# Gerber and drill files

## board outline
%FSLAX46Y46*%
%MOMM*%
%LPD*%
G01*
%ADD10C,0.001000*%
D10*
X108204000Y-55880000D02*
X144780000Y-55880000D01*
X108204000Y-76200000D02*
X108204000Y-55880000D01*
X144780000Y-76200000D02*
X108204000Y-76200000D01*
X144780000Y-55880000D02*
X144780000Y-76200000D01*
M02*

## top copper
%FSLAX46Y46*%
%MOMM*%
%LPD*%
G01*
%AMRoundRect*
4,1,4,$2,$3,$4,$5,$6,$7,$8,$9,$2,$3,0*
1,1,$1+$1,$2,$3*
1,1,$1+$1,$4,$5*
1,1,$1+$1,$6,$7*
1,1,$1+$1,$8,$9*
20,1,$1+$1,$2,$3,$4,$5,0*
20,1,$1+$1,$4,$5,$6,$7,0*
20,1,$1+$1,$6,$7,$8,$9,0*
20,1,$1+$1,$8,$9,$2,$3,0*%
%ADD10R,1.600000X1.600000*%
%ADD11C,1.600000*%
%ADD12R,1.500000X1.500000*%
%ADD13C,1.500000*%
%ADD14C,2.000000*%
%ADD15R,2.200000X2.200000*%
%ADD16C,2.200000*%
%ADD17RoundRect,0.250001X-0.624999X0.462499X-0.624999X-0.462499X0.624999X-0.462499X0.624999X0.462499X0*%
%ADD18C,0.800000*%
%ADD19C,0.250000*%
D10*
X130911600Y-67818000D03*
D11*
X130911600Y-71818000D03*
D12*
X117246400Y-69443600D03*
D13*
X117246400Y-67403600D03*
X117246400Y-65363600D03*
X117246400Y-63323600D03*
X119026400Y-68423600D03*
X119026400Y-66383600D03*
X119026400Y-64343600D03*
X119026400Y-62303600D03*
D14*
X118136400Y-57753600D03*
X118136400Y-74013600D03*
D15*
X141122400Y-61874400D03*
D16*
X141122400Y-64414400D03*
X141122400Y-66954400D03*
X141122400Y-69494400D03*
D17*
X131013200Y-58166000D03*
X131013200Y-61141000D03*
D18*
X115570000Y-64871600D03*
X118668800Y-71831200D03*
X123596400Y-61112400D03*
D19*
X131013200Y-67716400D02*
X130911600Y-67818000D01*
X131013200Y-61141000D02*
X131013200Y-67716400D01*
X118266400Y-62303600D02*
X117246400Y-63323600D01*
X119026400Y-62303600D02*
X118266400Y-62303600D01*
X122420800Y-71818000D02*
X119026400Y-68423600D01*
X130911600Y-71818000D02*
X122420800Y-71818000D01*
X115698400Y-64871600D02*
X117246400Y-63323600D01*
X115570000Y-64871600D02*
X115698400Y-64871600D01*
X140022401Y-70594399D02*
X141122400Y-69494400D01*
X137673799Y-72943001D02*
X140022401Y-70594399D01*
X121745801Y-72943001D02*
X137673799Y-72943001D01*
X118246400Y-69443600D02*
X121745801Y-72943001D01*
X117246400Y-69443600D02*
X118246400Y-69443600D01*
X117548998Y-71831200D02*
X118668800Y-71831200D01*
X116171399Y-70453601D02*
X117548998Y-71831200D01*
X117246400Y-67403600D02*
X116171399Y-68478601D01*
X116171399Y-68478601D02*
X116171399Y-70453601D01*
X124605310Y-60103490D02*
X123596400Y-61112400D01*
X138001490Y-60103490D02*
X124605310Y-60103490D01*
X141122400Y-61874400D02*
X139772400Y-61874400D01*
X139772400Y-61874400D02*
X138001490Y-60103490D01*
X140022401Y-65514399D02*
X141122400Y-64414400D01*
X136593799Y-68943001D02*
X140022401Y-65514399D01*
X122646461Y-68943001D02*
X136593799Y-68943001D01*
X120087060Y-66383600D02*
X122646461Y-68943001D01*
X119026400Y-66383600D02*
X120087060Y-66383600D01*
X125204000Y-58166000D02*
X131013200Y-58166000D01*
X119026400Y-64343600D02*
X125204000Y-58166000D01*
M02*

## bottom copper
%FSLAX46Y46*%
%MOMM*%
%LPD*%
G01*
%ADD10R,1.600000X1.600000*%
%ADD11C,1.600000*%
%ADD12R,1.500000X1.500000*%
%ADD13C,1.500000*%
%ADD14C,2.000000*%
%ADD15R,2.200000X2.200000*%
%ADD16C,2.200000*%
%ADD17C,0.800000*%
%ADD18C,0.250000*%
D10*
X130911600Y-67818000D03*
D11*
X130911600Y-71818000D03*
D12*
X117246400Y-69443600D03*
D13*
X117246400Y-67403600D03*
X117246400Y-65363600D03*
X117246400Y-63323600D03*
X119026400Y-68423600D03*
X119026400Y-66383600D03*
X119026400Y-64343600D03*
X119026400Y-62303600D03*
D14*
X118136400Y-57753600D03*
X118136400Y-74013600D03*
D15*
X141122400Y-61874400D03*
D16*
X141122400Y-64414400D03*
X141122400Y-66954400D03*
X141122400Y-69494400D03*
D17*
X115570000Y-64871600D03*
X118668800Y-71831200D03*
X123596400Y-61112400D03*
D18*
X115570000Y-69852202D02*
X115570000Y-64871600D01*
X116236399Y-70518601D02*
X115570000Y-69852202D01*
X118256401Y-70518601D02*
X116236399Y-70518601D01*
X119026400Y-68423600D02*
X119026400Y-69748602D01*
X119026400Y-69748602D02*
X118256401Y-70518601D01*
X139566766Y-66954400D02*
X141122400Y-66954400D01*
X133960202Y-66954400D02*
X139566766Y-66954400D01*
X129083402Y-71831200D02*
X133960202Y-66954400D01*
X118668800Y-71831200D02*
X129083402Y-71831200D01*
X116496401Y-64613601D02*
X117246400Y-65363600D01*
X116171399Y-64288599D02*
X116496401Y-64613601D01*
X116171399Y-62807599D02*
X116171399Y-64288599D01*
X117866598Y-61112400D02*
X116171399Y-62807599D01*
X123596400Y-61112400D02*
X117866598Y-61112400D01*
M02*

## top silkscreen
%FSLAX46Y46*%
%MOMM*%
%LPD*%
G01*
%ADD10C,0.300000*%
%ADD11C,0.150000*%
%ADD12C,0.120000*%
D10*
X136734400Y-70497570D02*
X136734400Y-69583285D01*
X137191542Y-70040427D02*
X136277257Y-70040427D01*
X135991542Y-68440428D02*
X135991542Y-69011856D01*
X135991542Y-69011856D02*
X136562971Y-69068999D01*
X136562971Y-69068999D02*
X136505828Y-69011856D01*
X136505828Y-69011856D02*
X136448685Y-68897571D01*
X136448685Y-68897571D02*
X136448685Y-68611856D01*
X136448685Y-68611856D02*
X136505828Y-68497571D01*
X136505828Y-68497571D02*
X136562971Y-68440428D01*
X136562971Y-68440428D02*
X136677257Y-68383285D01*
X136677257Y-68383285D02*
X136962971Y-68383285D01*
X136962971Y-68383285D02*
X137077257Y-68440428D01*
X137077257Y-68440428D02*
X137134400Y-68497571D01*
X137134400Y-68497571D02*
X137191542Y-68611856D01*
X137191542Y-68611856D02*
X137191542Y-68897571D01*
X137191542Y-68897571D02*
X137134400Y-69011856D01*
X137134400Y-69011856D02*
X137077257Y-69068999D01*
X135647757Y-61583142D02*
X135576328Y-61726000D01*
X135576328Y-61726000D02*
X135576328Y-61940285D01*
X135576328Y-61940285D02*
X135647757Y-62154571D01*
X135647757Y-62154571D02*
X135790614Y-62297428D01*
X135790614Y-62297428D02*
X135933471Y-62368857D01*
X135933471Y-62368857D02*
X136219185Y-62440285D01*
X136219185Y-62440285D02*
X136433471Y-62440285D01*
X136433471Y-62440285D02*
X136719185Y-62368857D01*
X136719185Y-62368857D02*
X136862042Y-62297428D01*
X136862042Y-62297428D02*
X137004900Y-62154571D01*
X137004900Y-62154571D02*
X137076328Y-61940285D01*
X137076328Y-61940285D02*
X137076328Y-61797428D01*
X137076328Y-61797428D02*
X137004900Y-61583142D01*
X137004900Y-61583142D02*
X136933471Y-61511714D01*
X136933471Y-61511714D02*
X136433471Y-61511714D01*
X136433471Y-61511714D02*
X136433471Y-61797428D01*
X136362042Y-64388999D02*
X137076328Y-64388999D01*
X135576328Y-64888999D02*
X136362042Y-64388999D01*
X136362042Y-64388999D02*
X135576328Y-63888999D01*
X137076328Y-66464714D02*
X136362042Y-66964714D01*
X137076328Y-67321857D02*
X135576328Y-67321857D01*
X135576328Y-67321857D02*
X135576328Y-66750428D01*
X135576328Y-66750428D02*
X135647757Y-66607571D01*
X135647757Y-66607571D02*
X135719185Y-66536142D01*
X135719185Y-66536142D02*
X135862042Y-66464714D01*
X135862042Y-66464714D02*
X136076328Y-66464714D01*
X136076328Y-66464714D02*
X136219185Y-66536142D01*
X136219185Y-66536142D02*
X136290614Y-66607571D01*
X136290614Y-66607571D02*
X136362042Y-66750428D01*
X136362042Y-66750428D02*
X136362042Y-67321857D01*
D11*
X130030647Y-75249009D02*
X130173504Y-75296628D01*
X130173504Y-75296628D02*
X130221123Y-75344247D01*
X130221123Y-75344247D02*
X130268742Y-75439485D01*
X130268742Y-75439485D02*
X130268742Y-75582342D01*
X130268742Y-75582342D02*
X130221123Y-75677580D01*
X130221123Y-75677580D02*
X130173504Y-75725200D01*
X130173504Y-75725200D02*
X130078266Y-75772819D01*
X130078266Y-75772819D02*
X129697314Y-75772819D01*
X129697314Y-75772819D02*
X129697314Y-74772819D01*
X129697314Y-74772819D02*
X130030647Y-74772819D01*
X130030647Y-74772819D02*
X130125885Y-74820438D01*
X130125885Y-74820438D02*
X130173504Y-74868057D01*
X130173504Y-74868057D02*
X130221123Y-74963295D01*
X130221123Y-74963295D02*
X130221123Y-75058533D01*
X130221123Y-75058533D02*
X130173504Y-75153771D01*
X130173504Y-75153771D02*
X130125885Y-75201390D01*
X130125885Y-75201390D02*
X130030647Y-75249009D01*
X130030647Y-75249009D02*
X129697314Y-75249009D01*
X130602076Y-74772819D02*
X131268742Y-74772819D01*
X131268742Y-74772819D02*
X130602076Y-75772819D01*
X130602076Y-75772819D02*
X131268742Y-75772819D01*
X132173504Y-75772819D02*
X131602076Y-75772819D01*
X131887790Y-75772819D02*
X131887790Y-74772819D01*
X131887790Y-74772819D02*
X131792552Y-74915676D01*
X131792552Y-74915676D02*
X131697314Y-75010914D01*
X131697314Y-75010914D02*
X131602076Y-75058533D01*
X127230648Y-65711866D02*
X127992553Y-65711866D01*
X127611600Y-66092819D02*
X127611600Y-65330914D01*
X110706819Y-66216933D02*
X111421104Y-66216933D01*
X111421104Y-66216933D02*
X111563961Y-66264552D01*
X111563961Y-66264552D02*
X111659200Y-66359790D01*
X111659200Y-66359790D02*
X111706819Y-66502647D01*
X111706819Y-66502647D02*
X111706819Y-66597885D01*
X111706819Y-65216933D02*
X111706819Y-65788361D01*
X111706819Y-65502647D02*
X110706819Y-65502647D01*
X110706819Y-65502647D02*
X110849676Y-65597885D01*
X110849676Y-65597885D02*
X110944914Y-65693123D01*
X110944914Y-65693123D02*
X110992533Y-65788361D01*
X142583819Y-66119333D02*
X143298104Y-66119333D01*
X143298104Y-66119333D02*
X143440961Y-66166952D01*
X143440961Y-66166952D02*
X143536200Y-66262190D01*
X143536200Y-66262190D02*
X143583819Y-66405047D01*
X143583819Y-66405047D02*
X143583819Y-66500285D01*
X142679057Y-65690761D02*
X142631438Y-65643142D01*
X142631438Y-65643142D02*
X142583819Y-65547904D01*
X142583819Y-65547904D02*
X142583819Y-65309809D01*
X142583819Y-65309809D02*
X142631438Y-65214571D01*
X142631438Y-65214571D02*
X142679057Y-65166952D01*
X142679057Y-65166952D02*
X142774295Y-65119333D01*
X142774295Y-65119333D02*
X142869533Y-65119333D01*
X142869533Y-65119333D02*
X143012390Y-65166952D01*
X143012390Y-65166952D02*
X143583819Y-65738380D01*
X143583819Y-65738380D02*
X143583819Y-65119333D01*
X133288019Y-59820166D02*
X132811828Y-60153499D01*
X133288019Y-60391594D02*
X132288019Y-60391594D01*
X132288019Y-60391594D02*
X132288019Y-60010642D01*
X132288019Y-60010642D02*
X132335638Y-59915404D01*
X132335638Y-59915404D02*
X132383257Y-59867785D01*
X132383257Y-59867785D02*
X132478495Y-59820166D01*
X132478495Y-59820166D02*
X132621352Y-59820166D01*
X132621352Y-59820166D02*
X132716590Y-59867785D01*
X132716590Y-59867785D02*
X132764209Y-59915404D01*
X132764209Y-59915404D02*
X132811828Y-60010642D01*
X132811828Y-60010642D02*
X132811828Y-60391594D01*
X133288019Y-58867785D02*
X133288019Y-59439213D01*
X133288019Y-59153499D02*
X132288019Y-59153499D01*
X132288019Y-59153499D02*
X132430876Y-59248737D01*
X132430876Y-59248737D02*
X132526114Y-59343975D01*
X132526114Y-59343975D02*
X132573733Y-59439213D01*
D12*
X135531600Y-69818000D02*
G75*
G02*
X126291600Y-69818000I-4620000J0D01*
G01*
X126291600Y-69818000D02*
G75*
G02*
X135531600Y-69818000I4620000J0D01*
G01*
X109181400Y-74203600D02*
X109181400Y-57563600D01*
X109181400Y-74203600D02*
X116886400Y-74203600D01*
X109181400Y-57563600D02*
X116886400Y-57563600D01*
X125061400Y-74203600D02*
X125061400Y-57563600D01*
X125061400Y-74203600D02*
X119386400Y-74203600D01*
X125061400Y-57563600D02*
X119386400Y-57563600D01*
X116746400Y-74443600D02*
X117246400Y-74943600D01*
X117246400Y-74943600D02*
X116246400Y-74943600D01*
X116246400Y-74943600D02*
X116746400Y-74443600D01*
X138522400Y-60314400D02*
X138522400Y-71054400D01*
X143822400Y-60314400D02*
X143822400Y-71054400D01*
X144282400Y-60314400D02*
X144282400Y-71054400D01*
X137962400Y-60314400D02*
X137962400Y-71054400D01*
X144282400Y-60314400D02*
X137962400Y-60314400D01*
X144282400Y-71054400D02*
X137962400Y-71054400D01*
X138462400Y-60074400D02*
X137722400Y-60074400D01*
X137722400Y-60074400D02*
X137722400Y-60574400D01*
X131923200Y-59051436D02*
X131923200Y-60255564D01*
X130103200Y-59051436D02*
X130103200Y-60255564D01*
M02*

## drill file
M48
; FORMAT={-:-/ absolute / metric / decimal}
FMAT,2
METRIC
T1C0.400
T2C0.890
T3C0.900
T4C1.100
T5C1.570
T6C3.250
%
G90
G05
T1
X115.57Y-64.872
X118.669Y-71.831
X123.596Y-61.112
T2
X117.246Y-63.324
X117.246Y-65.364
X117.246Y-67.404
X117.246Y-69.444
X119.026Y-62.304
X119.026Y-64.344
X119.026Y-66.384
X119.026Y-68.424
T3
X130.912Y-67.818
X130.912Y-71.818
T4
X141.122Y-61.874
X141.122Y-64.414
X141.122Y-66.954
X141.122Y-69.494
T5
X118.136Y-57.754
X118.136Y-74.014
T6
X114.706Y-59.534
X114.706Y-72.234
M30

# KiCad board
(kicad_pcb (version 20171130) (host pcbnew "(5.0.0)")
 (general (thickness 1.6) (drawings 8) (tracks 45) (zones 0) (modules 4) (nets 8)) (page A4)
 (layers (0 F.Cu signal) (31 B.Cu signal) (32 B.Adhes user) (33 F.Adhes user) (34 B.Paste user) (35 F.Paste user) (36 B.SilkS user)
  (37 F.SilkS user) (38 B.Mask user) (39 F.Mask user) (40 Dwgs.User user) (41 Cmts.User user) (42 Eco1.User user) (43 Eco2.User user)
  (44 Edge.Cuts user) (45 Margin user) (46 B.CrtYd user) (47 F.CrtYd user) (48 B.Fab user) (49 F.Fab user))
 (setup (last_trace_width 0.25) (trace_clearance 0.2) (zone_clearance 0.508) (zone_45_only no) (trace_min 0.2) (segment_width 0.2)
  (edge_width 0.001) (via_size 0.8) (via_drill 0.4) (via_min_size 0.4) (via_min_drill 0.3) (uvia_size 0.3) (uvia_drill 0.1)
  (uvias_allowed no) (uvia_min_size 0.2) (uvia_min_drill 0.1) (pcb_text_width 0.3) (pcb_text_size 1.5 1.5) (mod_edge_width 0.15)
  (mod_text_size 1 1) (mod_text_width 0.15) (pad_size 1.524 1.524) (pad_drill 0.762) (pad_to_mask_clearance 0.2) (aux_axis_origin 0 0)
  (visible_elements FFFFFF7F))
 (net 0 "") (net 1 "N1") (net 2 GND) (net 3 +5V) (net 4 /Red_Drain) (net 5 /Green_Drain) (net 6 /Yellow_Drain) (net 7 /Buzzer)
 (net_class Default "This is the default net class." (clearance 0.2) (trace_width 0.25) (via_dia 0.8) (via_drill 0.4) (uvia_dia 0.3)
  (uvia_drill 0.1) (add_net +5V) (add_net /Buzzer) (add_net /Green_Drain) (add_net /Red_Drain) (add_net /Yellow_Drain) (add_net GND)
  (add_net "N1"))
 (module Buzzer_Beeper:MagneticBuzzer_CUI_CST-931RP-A (layer F.Cu) (at 130.9116 67.818)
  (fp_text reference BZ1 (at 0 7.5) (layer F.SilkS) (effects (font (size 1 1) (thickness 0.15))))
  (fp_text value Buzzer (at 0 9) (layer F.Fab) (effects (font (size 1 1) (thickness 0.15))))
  (fp_circle (center 0 2) (end 4.62 2) (layer F.SilkS) (width 0.12))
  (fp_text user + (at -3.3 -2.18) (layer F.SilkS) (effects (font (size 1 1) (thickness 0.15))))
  (pad 1 thru_hole rect (at 0 0) (size 1.6 1.6) (drill 0.9) (layers *.Cu *.Mask) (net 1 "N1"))
  (pad 2 thru_hole circle (at 0 4) (size 1.6 1.6) (drill 0.9) (layers *.Cu *.Mask) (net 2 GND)))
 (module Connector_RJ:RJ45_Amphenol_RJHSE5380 (layer F.Cu) (at 117.2464 69.4436 90)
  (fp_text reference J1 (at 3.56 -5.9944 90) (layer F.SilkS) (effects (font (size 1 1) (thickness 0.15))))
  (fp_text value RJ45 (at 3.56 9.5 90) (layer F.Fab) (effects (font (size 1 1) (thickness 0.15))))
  (fp_line (start -4.76 -8.065) (end 11.88 -8.065) (layer F.SilkS) (width 0.12))
  (fp_line (start -4.76 -8.065) (end -4.76 -0.36) (layer F.SilkS) (width 0.12))
  (fp_line (start 11.88 -8.065) (end 11.88 -0.36) (layer F.SilkS) (width 0.12))
  (fp_line (start -4.76 7.815) (end 11.88 7.815) (layer F.SilkS) (width 0.12))
  (fp_line (start -4.76 7.815) (end -4.76 2.14) (layer F.SilkS) (width 0.12))
  (fp_line (start 11.88 7.815) (end 11.88 2.14) (layer F.SilkS) (width 0.12))
  (fp_line (start -5 -0.5) (end -5.5 0) (layer F.SilkS) (width 0.12))
  (fp_line (start -5.5 0) (end -5.5 -1) (layer F.SilkS) (width 0.12))
  (fp_line (start -5.5 -1) (end -5 -0.5) (layer F.SilkS) (width 0.12))
  (pad 1 thru_hole rect (at 0 0 90) (size 1.5 1.5) (drill 0.89) (layers *.Cu *.Mask) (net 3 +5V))
  (pad 3 thru_hole circle (at 2.04 0 90) (size 1.5 1.5) (drill 0.89) (layers *.Cu *.Mask) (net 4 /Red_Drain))
  (pad 5 thru_hole circle (at 4.08 0 90) (size 1.5 1.5) (drill 0.89) (layers *.Cu *.Mask) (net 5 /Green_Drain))
  (pad 7 thru_hole circle (at 6.12 0 90) (size 1.5 1.5) (drill 0.89) (layers *.Cu *.Mask) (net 2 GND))
  (pad 2 thru_hole circle (at 1.02 1.78 90) (size 1.5 1.5) (drill 0.89) (layers *.Cu *.Mask) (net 2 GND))
  (pad 4 thru_hole circle (at 3.06 1.78 90) (size 1.5 1.5) (drill 0.89) (layers *.Cu *.Mask) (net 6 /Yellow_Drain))
  (pad 6 thru_hole circle (at 5.1 1.78 90) (size 1.5 1.5) (drill 0.89) (layers *.Cu *.Mask) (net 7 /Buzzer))
  (pad 8 thru_hole circle (at 7.14 1.78 90) (size 1.5 1.5) (drill 0.89) (layers *.Cu *.Mask) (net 2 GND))
  (pad "" np_thru_hole circle (at -2.79 -2.54 90) (size 3.25 3.25) (drill 3.25) (layers *.Cu *.Mask))
  (pad "" np_thru_hole circle (at 9.91 -2.54 90) (size 3.25 3.25) (drill 3.25) (layers *.Cu *.Mask))
  (pad SH thru_hole circle (at 11.69 0.89 90) (size 2 2) (drill 1.57) (layers *.Cu *.Mask))
  (pad SH thru_hole circle (at -4.57 0.89 90) (size 2 2) (drill 1.57) (layers *.Cu *.Mask)))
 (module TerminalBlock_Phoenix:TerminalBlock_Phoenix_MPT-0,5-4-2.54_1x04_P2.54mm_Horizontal (layer F.Cu) (at 141.1224 61.8744 270)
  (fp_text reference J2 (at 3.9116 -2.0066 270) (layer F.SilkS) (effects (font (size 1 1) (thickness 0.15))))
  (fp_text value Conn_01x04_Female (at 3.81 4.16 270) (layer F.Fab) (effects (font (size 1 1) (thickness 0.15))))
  (fp_line (start -1.56 2.6) (end 9.18 2.6) (layer F.SilkS) (width 0.12))
  (fp_line (start -1.56 -2.7) (end 9.18 -2.7) (layer F.SilkS) (width 0.12))
  (fp_line (start -1.56 -3.16) (end 9.18 -3.16) (layer F.SilkS) (width 0.12))
  (fp_line (start -1.56 3.16) (end 9.18 3.16) (layer F.SilkS) (width 0.12))
  (fp_line (start -1.56 -3.16) (end -1.56 3.16) (layer F.SilkS) (width 0.12))
  (fp_line (start 9.18 -3.16) (end 9.18 3.16) (layer F.SilkS) (width 0.12))
  (fp_line (start -1.8 2.66) (end -1.8 3.4) (layer F.SilkS) (width 0.12))
  (fp_line (start -1.8 3.4) (end -1.3 3.4) (layer F.SilkS) (width 0.12))
  (pad 1 thru_hole rect (at 0 0 270) (size 2.2 2.2) (drill 1.1) (layers *.Cu *.Mask) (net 5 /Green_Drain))
  (pad 2 thru_hole circle (at 2.54 0 270) (size 2.2 2.2) (drill 1.1) (layers *.Cu *.Mask) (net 6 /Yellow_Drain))
  (pad 3 thru_hole circle (at 5.08 0 270) (size 2.2 2.2) (drill 1.1) (layers *.Cu *.Mask) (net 4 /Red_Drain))
  (pad 4 thru_hole circle (at 7.62 0 270) (size 2.2 2.2) (drill 1.1) (layers *.Cu *.Mask) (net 3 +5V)))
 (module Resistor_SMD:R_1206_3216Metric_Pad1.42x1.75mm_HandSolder (layer F.Cu) (at 131.0132 59.6535 270)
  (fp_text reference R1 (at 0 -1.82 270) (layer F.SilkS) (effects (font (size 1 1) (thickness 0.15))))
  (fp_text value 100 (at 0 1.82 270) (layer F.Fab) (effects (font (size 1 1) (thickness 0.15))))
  (fp_line (start -0.602064 -0.91) (end 0.602064 -0.91) (layer F.SilkS) (width 0.12))
  (fp_line (start -0.602064 0.91) (end 0.602064 0.91) (layer F.SilkS) (width 0.12))
  (pad 1 smd roundrect (at -1.4875 0 270) (size 1.425 1.75) (layers F.Cu F.Paste F.Mask) (roundrect_rratio 0.175439) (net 7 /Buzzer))
  (pad 2 smd roundrect (at 1.4875 0 270) (size 1.425 1.75) (layers F.Cu F.Paste F.Mask) (roundrect_rratio 0.175439) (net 1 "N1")))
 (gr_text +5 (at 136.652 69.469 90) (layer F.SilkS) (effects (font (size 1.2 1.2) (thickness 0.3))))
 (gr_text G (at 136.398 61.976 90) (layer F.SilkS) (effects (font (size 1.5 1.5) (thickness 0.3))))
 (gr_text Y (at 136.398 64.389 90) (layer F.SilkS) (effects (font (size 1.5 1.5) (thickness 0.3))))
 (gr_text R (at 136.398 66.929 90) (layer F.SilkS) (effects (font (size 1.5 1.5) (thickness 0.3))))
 (gr_line (start 108.204 55.88) (end 144.78 55.88) (layer Edge.Cuts) (width 0.001))
 (gr_line (start 108.204 76.2) (end 108.204 55.88) (layer Edge.Cuts) (width 0.001))
 (gr_line (start 144.78 76.2) (end 108.204 76.2) (layer Edge.Cuts) (width 0.001))
 (gr_line (start 144.78 55.88) (end 144.78 76.2) (layer Edge.Cuts) (width 0.001))
 (segment (start 131.0132 67.7164) (end 130.9116 67.818) (width 0.25) (layer F.Cu) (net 1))
 (segment (start 131.0132 61.141) (end 131.0132 67.7164) (width 0.25) (layer F.Cu) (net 1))
 (segment (start 118.2664 62.3036) (end 117.2464 63.3236) (width 0.25) (layer F.Cu) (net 2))
 (segment (start 119.0264 62.3036) (end 118.2664 62.3036) (width 0.25) (layer F.Cu) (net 2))
 (segment (start 122.4208 71.818) (end 119.0264 68.4236) (width 0.25) (layer F.Cu) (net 2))
 (segment (start 130.9116 71.818) (end 122.4208 71.818) (width 0.25) (layer F.Cu) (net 2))
 (via (at 115.57 64.8716) (size 0.8) (drill 0.4) (layers F.Cu B.Cu) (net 2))
 (segment (start 115.57 69.852202) (end 115.57 64.8716) (width 0.25) (layer B.Cu) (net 2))
 (segment (start 116.236399 70.518601) (end 115.57 69.852202) (width 0.25) (layer B.Cu) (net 2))
 (segment (start 118.256401 70.518601) (end 116.236399 70.518601) (width 0.25) (layer B.Cu) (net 2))
 (segment (start 119.0264 68.4236) (end 119.0264 69.748602) (width 0.25) (layer B.Cu) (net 2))
 (segment (start 119.0264 69.748602) (end 118.256401 70.518601) (width 0.25) (layer B.Cu) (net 2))
 (segment (start 115.6984 64.8716) (end 117.2464 63.3236) (width 0.25) (layer F.Cu) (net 2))
 (segment (start 115.57 64.8716) (end 115.6984 64.8716) (width 0.25) (layer F.Cu) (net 2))
 (segment (start 140.022401 70.594399) (end 141.1224 69.4944) (width 0.25) (layer F.Cu) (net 3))
 (segment (start 137.673799 72.943001) (end 140.022401 70.594399) (width 0.25) (layer F.Cu) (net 3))
 (segment (start 121.745801 72.943001) (end 137.673799 72.943001) (width 0.25) (layer F.Cu) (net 3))
 (segment (start 118.2464 69.4436) (end 121.745801 72.943001) (width 0.25) (layer F.Cu) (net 3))
 (segment (start 117.2464 69.4436) (end 118.2464 69.4436) (width 0.25) (layer F.Cu) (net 3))
 (via (at 118.6688 71.8312) (size 0.8) (drill 0.4) (layers F.Cu B.Cu) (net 4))
 (segment (start 117.548998 71.8312) (end 118.6688 71.8312) (width 0.25) (layer F.Cu) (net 4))
 (segment (start 116.171399 70.453601) (end 117.548998 71.8312) (width 0.25) (layer F.Cu) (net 4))
 (segment (start 117.2464 67.4036) (end 116.171399 68.478601) (width 0.25) (layer F.Cu) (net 4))
 (segment (start 116.171399 68.478601) (end 116.171399 70.453601) (width 0.25) (layer F.Cu) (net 4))
 (segment (start 139.566766 66.9544) (end 141.1224 66.9544) (width 0.25) (layer B.Cu) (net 4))
 (segment (start 133.960202 66.9544) (end 139.566766 66.9544) (width 0.25) (layer B.Cu) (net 4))
 (segment (start 129.083402 71.8312) (end 133.960202 66.9544) (width 0.25) (layer B.Cu) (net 4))
 (segment (start 118.6688 71.8312) (end 129.083402 71.8312) (width 0.25) (layer B.Cu) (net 4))
 (via (at 123.5964 61.1124) (size 0.8) (drill 0.4) (layers F.Cu B.Cu) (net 5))
 (segment (start 124.60531 60.10349) (end 123.5964 61.1124) (width 0.25) (layer F.Cu) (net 5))
 (segment (start 138.00149 60.10349) (end 124.60531 60.10349) (width 0.25) (layer F.Cu) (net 5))
 (segment (start 141.1224 61.8744) (end 139.7724 61.8744) (width 0.25) (layer F.Cu) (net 5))
 (segment (start 139.7724 61.8744) (end 138.00149 60.10349) (width 0.25) (layer F.Cu) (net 5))
 (segment (start 116.496401 64.613601) (end 117.2464 65.3636) (width 0.25) (layer B.Cu) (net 5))
 (segment (start 116.171399 64.288599) (end 116.496401 64.613601) (width 0.25) (layer B.Cu) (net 5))
 (segment (start 116.171399 62.807599) (end 116.171399 64.288599) (width 0.25) (layer B.Cu) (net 5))
 (segment (start 117.866598 61.1124) (end 116.171399 62.807599) (width 0.25) (layer B.Cu) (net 5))
 (segment (start 123.5964 61.1124) (end 117.866598 61.1124) (width 0.25) (layer B.Cu) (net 5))
 (segment (start 140.022401 65.514399) (end 141.1224 64.4144) (width 0.25) (layer F.Cu) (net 6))
 (segment (start 136.593799 68.943001) (end 140.022401 65.514399) (width 0.25) (layer F.Cu) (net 6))
 (segment (start 122.646461 68.943001) (end 136.593799 68.943001) (width 0.25) (layer F.Cu) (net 6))
 (segment (start 120.08706 66.3836) (end 122.646461 68.943001) (width 0.25) (layer F.Cu) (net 6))
 (segment (start 119.0264 66.3836) (end 120.08706 66.3836) (width 0.25) (layer F.Cu) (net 6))
 (segment (start 125.204 58.166) (end 131.0132 58.166) (width 0.25) (layer F.Cu) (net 7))
 (segment (start 119.0264 64.3436) (end 125.204 58.166) (width 0.25) (layer F.Cu) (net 7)))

